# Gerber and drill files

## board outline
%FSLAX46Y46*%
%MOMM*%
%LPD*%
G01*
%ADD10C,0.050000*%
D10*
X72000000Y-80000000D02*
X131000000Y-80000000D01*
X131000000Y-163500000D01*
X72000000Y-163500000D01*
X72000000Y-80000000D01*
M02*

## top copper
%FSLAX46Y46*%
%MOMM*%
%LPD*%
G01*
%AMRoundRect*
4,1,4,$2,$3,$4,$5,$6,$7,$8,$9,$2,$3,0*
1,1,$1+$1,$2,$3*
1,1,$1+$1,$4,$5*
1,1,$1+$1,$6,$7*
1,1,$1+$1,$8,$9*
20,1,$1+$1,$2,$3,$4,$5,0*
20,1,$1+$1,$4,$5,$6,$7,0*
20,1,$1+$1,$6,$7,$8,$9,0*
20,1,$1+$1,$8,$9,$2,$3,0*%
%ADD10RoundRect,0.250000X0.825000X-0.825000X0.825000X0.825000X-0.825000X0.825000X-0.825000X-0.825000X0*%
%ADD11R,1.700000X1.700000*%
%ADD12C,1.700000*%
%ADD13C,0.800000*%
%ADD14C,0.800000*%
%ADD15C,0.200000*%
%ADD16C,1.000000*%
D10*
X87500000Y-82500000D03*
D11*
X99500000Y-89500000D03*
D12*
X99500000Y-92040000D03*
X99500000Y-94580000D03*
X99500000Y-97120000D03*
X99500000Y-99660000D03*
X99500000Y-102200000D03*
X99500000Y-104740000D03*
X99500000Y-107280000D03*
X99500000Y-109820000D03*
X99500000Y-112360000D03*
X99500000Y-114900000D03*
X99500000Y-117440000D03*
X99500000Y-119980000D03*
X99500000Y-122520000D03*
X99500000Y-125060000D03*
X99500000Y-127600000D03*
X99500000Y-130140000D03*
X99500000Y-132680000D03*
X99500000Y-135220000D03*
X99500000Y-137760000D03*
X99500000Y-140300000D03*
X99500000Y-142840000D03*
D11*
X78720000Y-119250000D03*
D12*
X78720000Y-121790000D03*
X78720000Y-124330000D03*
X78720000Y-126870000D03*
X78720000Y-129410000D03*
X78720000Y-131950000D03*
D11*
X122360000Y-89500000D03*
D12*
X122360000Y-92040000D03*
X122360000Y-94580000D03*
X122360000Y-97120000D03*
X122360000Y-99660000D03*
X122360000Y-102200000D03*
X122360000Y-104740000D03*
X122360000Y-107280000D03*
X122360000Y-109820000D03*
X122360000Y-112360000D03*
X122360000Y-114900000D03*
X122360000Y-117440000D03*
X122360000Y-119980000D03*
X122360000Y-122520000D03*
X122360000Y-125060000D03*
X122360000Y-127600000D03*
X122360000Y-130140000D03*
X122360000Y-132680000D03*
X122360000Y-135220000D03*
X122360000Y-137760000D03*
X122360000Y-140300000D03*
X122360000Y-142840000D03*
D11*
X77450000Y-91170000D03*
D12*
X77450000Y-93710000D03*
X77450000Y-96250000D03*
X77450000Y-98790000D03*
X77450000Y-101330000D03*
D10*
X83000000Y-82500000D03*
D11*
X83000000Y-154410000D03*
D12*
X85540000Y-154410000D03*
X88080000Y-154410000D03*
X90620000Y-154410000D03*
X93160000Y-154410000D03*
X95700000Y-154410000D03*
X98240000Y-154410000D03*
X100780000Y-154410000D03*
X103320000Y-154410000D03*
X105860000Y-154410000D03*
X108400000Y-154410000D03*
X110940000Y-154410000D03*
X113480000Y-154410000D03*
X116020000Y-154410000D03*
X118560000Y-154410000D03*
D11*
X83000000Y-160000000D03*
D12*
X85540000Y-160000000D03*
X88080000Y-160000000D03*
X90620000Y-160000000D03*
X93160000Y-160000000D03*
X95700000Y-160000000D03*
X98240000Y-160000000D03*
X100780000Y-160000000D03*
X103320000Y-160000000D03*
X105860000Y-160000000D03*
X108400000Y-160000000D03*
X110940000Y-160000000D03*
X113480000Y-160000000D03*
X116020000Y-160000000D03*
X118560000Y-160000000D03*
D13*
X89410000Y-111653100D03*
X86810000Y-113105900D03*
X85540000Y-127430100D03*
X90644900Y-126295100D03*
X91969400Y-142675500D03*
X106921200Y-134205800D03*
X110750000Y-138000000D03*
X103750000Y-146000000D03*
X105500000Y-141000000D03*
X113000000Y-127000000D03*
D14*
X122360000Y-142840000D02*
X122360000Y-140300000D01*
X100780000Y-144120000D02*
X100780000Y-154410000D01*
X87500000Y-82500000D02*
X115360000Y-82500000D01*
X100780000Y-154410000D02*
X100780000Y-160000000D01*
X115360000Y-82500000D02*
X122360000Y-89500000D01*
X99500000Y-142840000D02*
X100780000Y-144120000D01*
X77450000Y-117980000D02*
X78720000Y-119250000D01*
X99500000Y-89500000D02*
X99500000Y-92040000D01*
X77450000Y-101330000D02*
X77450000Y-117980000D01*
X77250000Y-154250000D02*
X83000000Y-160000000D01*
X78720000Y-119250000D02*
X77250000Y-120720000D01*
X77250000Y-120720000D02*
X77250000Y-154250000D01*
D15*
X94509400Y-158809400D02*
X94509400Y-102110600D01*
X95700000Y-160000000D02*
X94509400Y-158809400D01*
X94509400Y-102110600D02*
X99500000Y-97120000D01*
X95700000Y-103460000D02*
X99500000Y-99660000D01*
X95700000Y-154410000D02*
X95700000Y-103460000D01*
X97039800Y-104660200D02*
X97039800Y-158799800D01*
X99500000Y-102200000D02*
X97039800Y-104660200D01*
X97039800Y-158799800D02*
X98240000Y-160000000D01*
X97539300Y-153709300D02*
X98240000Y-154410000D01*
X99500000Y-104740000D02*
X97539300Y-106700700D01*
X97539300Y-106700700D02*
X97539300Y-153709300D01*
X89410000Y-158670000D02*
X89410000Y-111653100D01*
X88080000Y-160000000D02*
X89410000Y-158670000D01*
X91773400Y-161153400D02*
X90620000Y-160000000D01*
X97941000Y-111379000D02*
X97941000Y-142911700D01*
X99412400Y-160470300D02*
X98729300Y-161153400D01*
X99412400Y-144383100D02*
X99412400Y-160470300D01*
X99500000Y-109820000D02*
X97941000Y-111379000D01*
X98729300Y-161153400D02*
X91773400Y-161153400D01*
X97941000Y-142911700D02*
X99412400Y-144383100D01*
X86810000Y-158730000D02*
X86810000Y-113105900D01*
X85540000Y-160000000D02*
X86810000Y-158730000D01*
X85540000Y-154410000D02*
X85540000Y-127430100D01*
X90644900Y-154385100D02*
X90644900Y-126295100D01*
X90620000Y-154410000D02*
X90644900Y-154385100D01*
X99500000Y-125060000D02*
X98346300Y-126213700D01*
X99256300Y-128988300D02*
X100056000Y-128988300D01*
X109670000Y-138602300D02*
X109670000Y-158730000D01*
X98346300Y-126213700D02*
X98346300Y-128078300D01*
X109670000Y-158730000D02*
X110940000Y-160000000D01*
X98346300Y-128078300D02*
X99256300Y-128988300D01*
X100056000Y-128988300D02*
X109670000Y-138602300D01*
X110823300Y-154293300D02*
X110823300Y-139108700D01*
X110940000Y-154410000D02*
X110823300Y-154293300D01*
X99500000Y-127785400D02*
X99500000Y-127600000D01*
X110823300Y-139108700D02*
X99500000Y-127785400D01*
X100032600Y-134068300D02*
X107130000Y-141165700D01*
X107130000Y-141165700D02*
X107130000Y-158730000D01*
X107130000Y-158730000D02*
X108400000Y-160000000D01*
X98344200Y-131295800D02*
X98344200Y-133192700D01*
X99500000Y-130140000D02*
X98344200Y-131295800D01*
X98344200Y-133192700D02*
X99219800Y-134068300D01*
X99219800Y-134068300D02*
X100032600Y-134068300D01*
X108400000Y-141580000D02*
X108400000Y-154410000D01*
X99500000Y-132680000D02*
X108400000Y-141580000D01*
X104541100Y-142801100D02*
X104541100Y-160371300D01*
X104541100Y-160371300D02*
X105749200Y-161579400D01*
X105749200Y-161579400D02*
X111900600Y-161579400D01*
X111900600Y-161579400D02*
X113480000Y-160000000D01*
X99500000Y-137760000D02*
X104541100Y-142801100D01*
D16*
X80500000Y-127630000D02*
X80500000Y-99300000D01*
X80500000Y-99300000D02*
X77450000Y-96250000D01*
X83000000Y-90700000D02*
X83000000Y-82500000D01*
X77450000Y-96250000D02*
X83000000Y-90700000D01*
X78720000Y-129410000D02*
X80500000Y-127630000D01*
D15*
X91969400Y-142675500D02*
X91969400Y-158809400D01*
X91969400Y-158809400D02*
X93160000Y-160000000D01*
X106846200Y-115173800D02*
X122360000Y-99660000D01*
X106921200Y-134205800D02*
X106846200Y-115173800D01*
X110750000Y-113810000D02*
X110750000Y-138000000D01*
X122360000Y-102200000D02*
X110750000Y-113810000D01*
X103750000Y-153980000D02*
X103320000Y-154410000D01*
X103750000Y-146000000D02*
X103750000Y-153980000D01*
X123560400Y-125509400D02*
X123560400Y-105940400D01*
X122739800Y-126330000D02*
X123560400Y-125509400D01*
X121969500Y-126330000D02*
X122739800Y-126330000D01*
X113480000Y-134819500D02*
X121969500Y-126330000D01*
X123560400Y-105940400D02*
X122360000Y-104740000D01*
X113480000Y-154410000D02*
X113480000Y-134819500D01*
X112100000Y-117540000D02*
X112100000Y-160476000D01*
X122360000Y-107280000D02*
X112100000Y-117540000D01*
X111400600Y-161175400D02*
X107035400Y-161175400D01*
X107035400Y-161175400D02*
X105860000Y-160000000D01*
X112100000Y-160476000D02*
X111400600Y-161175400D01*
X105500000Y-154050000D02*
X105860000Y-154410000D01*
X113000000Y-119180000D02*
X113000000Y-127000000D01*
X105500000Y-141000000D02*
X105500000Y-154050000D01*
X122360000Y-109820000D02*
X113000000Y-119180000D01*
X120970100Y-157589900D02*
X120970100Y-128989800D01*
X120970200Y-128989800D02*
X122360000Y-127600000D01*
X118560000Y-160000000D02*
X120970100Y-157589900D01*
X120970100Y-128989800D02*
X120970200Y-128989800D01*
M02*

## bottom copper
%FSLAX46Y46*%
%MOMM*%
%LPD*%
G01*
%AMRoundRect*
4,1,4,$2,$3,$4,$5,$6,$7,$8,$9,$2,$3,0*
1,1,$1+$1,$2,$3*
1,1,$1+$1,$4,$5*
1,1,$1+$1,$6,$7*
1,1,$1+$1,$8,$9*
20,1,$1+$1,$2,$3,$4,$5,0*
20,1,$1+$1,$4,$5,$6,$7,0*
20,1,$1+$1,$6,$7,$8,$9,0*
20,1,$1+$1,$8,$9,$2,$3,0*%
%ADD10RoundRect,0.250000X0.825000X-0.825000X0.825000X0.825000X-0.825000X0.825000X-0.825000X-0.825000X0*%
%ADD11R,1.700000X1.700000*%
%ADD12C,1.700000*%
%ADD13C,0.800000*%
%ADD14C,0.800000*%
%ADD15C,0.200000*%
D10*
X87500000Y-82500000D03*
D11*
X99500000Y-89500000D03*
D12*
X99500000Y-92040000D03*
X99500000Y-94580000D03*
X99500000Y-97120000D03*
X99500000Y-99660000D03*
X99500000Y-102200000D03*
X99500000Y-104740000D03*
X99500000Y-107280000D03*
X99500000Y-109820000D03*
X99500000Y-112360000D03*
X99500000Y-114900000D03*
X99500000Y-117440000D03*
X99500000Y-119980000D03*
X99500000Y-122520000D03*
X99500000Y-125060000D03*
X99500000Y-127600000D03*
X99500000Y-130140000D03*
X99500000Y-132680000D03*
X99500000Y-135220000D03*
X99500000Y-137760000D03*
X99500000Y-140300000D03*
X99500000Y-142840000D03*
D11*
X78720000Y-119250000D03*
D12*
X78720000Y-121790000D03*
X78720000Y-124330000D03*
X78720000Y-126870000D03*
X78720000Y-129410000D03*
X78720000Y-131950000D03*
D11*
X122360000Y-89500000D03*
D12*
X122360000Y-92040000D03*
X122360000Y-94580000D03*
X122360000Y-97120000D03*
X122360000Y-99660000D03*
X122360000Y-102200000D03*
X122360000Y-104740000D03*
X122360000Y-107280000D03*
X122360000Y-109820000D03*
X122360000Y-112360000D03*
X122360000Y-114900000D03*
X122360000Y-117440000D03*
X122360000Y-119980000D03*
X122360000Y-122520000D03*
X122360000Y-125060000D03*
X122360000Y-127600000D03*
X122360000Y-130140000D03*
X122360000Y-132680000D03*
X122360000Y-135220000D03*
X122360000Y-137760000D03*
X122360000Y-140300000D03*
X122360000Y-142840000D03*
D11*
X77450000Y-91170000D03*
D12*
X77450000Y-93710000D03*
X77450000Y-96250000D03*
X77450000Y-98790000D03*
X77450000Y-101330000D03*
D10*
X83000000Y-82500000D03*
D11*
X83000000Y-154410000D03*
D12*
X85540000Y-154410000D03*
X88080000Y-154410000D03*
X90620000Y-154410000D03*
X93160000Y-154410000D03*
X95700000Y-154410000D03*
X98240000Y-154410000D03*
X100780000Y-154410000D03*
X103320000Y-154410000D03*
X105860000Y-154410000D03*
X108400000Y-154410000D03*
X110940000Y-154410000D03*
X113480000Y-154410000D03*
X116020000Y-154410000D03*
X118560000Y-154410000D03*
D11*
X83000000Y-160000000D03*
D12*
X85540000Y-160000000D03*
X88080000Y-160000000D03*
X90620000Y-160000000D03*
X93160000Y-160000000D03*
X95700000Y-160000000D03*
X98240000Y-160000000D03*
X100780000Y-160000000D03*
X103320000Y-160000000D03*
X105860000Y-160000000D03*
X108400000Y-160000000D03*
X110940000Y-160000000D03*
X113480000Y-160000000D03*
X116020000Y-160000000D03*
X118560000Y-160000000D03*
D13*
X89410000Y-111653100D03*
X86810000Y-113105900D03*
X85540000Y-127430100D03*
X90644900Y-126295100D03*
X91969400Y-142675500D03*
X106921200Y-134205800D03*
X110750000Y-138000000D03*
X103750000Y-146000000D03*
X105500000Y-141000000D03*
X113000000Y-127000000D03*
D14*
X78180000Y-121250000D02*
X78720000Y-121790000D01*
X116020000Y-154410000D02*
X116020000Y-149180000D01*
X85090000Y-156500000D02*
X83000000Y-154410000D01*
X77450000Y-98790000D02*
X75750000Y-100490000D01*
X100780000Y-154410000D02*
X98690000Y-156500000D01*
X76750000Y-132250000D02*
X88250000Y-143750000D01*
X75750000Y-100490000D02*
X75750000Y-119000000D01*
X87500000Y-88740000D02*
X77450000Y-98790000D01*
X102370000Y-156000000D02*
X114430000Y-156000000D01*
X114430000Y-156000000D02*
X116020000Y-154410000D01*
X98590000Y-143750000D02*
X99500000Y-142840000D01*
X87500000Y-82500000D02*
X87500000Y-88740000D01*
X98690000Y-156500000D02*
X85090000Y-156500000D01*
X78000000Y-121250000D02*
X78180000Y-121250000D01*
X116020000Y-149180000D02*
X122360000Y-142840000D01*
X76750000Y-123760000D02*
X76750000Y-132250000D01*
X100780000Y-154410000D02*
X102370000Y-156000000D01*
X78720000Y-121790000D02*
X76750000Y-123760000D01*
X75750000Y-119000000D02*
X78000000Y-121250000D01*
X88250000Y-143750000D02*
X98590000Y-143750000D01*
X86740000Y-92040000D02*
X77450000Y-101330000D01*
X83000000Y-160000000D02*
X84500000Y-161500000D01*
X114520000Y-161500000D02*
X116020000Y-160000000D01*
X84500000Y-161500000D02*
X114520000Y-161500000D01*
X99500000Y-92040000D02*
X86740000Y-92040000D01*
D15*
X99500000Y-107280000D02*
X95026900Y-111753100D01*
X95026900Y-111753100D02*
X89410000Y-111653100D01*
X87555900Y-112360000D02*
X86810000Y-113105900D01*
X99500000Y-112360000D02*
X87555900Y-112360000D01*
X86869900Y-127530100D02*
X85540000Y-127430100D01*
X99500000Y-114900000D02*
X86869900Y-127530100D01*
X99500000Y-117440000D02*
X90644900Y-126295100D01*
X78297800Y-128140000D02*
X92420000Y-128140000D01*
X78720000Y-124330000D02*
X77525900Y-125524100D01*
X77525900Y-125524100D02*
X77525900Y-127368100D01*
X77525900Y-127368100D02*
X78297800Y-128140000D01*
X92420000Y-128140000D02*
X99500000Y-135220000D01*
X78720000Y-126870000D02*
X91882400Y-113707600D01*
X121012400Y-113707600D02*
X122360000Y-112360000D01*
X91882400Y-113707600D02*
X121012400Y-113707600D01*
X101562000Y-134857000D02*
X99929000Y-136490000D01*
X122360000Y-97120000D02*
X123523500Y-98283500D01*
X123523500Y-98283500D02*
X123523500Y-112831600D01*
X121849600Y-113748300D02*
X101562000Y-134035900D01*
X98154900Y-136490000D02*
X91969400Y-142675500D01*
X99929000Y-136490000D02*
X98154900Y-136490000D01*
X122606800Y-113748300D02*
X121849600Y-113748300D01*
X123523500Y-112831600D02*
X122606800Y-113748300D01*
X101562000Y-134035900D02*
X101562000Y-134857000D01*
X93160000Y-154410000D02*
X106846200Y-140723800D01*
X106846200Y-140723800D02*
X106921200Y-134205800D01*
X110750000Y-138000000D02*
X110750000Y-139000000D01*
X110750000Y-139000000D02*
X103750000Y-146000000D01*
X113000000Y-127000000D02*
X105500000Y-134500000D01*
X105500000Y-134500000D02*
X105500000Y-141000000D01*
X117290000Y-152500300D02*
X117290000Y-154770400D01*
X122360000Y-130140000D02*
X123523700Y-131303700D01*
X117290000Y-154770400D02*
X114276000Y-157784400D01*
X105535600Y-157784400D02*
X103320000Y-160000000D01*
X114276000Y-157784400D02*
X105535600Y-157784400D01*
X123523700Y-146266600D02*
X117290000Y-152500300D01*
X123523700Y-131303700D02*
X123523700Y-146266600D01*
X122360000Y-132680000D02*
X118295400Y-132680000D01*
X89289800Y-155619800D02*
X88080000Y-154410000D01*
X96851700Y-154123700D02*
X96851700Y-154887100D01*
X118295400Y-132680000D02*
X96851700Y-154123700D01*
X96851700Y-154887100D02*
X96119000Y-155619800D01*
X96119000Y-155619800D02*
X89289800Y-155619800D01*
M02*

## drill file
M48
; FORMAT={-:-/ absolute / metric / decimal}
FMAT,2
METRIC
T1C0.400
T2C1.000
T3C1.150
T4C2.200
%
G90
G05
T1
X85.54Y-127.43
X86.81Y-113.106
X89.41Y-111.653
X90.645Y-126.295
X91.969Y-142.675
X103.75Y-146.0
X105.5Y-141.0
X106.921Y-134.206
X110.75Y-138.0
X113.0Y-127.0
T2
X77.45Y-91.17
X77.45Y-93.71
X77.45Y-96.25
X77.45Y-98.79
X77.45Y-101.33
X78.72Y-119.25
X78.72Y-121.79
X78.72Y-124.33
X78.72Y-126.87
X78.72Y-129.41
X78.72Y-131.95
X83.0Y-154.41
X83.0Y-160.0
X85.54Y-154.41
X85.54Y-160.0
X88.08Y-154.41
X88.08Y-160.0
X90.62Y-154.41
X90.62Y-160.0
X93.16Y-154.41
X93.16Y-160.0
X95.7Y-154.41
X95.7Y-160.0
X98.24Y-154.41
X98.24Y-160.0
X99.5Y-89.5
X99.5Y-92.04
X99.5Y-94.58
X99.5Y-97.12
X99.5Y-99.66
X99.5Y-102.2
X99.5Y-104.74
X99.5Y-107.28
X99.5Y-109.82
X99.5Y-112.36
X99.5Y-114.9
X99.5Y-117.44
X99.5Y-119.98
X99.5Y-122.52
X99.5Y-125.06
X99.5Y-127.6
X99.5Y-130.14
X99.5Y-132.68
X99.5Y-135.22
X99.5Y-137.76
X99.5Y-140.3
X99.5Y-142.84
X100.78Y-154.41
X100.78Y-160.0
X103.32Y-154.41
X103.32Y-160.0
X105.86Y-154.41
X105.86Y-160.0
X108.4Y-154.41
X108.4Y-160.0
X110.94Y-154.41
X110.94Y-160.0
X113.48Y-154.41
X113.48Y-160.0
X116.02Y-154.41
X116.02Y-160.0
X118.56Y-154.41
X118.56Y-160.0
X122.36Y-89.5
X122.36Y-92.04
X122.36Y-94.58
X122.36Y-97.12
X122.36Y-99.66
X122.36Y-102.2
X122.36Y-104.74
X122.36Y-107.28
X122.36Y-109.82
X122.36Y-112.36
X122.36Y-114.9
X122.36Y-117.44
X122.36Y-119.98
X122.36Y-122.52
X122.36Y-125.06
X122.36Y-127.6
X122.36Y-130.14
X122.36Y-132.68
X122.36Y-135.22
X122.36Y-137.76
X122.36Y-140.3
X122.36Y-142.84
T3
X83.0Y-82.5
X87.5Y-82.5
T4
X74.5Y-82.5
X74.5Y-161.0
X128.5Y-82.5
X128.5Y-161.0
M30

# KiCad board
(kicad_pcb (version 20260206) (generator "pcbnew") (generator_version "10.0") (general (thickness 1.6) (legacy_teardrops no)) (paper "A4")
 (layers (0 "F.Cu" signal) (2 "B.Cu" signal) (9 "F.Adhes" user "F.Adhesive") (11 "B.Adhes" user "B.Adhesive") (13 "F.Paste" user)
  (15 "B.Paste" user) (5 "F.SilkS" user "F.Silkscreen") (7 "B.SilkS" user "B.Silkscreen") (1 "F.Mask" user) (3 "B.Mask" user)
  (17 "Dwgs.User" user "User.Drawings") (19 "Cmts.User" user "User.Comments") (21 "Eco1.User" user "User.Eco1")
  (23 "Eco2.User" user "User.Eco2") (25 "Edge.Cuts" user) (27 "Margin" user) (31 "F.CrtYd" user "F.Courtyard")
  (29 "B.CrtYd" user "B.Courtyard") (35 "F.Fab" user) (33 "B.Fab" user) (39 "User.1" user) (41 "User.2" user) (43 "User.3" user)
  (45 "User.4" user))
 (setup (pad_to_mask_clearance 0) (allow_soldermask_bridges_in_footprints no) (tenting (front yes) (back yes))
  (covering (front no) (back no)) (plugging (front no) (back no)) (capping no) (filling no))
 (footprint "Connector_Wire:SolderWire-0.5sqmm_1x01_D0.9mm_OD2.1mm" (layer "F.Cu") (at 87.5 82.5 90)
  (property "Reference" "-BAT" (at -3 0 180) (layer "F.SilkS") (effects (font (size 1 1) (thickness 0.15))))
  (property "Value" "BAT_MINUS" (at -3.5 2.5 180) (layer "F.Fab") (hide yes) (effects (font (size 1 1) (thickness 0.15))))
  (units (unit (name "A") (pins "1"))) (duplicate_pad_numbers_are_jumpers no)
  (pad "1" thru_hole roundrect (at 0 0 90) (size 2.15 2.15) (drill 1.15) (layers "*.Cu" "*.Mask") (remove_unused_layers no)
   (roundrect_rratio 0.116279) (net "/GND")))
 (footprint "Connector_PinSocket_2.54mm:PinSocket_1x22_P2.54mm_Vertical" (layer "F.Cu") (at 99.5 89.5)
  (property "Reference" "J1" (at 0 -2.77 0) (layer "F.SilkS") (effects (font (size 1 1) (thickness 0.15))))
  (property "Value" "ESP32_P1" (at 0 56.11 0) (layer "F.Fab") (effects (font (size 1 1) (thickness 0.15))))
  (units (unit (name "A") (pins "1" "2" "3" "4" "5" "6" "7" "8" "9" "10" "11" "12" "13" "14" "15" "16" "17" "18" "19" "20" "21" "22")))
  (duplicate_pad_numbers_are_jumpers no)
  (pad "1" thru_hole rect (at 0 0) (size 1.7 1.7) (drill 1) (layers "*.Cu" "*.Mask") (remove_unused_layers no) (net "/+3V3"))
  (pad "2" thru_hole circle (at 0 2.54) (size 1.7 1.7) (drill 1) (layers "*.Cu" "*.Mask") (remove_unused_layers no) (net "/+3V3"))
  (pad "3" thru_hole circle (at 0 5.08) (size 1.7 1.7) (drill 1) (layers "*.Cu" "*.Mask") (remove_unused_layers no) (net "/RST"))
  (pad "4" thru_hole circle (at 0 7.62) (size 1.7 1.7) (drill 1) (layers "*.Cu" "*.Mask") (remove_unused_layers no) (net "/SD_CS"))
  (pad "5" thru_hole circle (at 0 10.16) (size 1.7 1.7) (drill 1) (layers "*.Cu" "*.Mask") (remove_unused_layers no) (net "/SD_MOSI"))
  (pad "6" thru_hole circle (at 0 12.7) (size 1.7 1.7) (drill 1) (layers "*.Cu" "*.Mask") (remove_unused_layers no) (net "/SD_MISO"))
  (pad "7" thru_hole circle (at 0 15.24) (size 1.7 1.7) (drill 1) (layers "*.Cu" "*.Mask") (remove_unused_layers no) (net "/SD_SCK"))
  (pad "8" thru_hole circle (at 0 17.78) (size 1.7 1.7) (drill 1) (layers "*.Cu" "*.Mask") (remove_unused_layers no) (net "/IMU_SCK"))
  (pad "9" thru_hole circle (at 0 20.32) (size 1.7 1.7) (drill 1) (layers "*.Cu" "*.Mask") (remove_unused_layers no) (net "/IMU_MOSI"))
  (pad "10" thru_hole circle (at 0 22.86) (size 1.7 1.7) (drill 1) (layers "*.Cu" "*.Mask") (remove_unused_layers no) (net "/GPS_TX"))
  (pad "11" thru_hole circle (at 0 25.4) (size 1.7 1.7) (drill 1) (layers "*.Cu" "*.Mask") (remove_unused_layers no) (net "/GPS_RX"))
  (pad "12" thru_hole circle (at 0 27.94) (size 1.7 1.7) (drill 1) (layers "*.Cu" "*.Mask") (remove_unused_layers no) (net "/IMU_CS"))
  (pad "13" thru_hole circle (at 0 30.48) (size 1.7 1.7) (drill 1) (layers "*.Cu" "*.Mask") (remove_unused_layers no) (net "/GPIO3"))
  (pad "14" thru_hole circle (at 0 33.02) (size 1.7 1.7) (drill 1) (layers "*.Cu" "*.Mask") (remove_unused_layers no) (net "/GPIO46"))
  (pad "15" thru_hole circle (at 0 35.56) (size 1.7 1.7) (drill 1) (layers "*.Cu" "*.Mask") (remove_unused_layers no) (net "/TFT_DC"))
  (pad "16" thru_hole circle (at 0 38.1) (size 1.7 1.7) (drill 1) (layers "*.Cu" "*.Mask") (remove_unused_layers no) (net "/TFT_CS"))
  (pad "17" thru_hole circle (at 0 40.64) (size 1.7 1.7) (drill 1) (layers "*.Cu" "*.Mask") (remove_unused_layers no) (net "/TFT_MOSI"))
  (pad "18" thru_hole circle (at 0 43.18) (size 1.7 1.7) (drill 1) (layers "*.Cu" "*.Mask") (remove_unused_layers no) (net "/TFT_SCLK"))
  (pad "19" thru_hole circle (at 0 45.72) (size 1.7 1.7) (drill 1) (layers "*.Cu" "*.Mask") (remove_unused_layers no) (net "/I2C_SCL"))
  (pad "20" thru_hole circle (at 0 48.26) (size 1.7 1.7) (drill 1) (layers "*.Cu" "*.Mask") (remove_unused_layers no) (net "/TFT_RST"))
  (pad "21" thru_hole circle (at 0 50.8) (size 1.7 1.7) (drill 1) (layers "*.Cu" "*.Mask") (remove_unused_layers no) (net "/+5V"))
  (pad "22" thru_hole circle (at 0 53.34) (size 1.7 1.7) (drill 1) (layers "*.Cu" "*.Mask") (remove_unused_layers no) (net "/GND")))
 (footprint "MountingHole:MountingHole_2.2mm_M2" (layer "F.Cu") (at 74.5 82.5)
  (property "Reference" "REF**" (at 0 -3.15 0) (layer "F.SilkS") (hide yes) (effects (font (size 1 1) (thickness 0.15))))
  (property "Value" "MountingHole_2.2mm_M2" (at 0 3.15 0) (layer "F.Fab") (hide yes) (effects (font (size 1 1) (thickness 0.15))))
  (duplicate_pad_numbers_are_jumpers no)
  (pad "" np_thru_hole circle (at 0 0) (size 2.2 2.2) (drill 2.2) (layers "*.Cu" "*.Mask")))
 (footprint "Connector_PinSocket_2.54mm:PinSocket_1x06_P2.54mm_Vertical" (layer "F.Cu") (at 78.72 119.25)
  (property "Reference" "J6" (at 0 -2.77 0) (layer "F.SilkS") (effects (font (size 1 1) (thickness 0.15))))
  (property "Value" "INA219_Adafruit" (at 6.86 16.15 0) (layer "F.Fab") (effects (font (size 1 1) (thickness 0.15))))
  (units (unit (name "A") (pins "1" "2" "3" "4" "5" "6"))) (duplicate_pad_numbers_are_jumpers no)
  (pad "1" thru_hole rect (at 0 0) (size 1.7 1.7) (drill 1) (layers "*.Cu" "*.Mask") (remove_unused_layers no) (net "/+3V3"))
  (pad "2" thru_hole circle (at 0 2.54) (size 1.7 1.7) (drill 1) (layers "*.Cu" "*.Mask") (remove_unused_layers no) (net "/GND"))
  (pad "3" thru_hole circle (at 0 5.08) (size 1.7 1.7) (drill 1) (layers "*.Cu" "*.Mask") (remove_unused_layers no) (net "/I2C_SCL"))
  (pad "4" thru_hole circle (at 0 7.62) (size 1.7 1.7) (drill 1) (layers "*.Cu" "*.Mask") (remove_unused_layers no) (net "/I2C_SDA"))
  (pad "5" thru_hole circle (at 0 10.16) (size 1.7 1.7) (drill 1) (layers "*.Cu" "*.Mask") (remove_unused_layers no) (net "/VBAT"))
  (pad "6" thru_hole circle (at 0 12.7) (size 1.7 1.7) (drill 1) (layers "*.Cu" "*.Mask") (remove_unused_layers no)
   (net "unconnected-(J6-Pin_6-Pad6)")))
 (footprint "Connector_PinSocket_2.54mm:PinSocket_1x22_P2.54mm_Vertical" (layer "F.Cu") (at 122.36 89.5)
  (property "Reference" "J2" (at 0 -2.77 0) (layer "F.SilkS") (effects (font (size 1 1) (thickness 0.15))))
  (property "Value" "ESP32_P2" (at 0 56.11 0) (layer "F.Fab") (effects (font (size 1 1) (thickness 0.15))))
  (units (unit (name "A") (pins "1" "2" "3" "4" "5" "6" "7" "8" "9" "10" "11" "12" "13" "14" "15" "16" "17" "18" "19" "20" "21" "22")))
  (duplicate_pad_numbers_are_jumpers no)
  (pad "1" thru_hole rect (at 0 0) (size 1.7 1.7) (drill 1) (layers "*.Cu" "*.Mask") (remove_unused_layers no) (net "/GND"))
  (pad "2" thru_hole circle (at 0 2.54) (size 1.7 1.7) (drill 1) (layers "*.Cu" "*.Mask") (remove_unused_layers no) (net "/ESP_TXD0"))
  (pad "3" thru_hole circle (at 0 5.08) (size 1.7 1.7) (drill 1) (layers "*.Cu" "*.Mask") (remove_unused_layers no) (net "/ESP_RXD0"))
  (pad "4" thru_hole circle (at 0 7.62) (size 1.7 1.7) (drill 1) (layers "*.Cu" "*.Mask") (remove_unused_layers no) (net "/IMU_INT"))
  (pad "5" thru_hole circle (at 0 10.16) (size 1.7 1.7) (drill 1) (layers "*.Cu" "*.Mask") (remove_unused_layers no) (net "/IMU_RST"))
  (pad "6" thru_hole circle (at 0 12.7) (size 1.7 1.7) (drill 1) (layers "*.Cu" "*.Mask") (remove_unused_layers no) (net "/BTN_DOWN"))
  (pad "7" thru_hole circle (at 0 15.24) (size 1.7 1.7) (drill 1) (layers "*.Cu" "*.Mask") (remove_unused_layers no) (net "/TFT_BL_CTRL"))
  (pad "8" thru_hole circle (at 0 17.78) (size 1.7 1.7) (drill 1) (layers "*.Cu" "*.Mask") (remove_unused_layers no) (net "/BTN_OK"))
  (pad "9" thru_hole circle (at 0 20.32) (size 1.7 1.7) (drill 1) (layers "*.Cu" "*.Mask") (remove_unused_layers no) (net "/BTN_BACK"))
  (pad "10" thru_hole circle (at 0 22.86) (size 1.7 1.7) (drill 1) (layers "*.Cu" "*.Mask") (remove_unused_layers no) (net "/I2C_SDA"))
  (pad "11" thru_hole circle (at 0 25.4) (size 1.7 1.7) (drill 1) (layers "*.Cu" "*.Mask") (remove_unused_layers no) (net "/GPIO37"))
  (pad "12" thru_hole circle (at 0 27.94) (size 1.7 1.7) (drill 1) (layers "*.Cu" "*.Mask") (remove_unused_layers no) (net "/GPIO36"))
  (pad "13" thru_hole circle (at 0 30.48) (size 1.7 1.7) (drill 1) (layers "*.Cu" "*.Mask") (remove_unused_layers no) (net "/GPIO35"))
  (pad "14" thru_hole circle (at 0 33.02) (size 1.7 1.7) (drill 1) (layers "*.Cu" "*.Mask") (remove_unused_layers no) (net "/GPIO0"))
  (pad "15" thru_hole circle (at 0 35.56) (size 1.7 1.7) (drill 1) (layers "*.Cu" "*.Mask") (remove_unused_layers no) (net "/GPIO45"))
  (pad "16" thru_hole circle (at 0 38.1) (size 1.7 1.7) (drill 1) (layers "*.Cu" "*.Mask") (remove_unused_layers no) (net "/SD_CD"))
  (pad "17" thru_hole circle (at 0 40.64) (size 1.7 1.7) (drill 1) (layers "*.Cu" "*.Mask") (remove_unused_layers no) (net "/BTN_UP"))
  (pad "18" thru_hole circle (at 0 43.18) (size 1.7 1.7) (drill 1) (layers "*.Cu" "*.Mask") (remove_unused_layers no) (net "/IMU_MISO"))
  (pad "19" thru_hole circle (at 0 45.72) (size 1.7 1.7) (drill 1) (layers "*.Cu" "*.Mask") (remove_unused_layers no) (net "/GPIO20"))
  (pad "20" thru_hole circle (at 0 48.26) (size 1.7 1.7) (drill 1) (layers "*.Cu" "*.Mask") (remove_unused_layers no) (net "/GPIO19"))
  (pad "21" thru_hole circle (at 0 50.8) (size 1.7 1.7) (drill 1) (layers "*.Cu" "*.Mask") (remove_unused_layers no) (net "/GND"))
  (pad "22" thru_hole circle (at 0 53.34) (size 1.7 1.7) (drill 1) (layers "*.Cu" "*.Mask") (remove_unused_layers no) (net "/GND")))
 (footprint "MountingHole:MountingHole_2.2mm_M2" (layer "F.Cu") (at 74.5 161)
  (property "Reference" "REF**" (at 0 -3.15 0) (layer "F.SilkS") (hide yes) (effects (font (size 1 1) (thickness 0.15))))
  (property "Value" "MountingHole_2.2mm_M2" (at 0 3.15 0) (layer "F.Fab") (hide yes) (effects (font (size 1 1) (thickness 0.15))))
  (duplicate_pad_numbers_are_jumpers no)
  (pad "" np_thru_hole circle (at 0 0) (size 2.2 2.2) (drill 2.2) (layers "*.Cu" "*.Mask")))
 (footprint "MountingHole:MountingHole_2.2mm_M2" (layer "F.Cu") (at 128.5 82.5)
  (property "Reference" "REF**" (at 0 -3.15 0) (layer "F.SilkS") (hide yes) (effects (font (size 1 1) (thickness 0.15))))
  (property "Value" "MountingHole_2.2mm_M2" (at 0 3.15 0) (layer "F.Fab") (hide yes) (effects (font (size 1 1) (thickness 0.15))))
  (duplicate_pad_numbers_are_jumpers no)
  (pad "" np_thru_hole circle (at 0 0) (size 2.2 2.2) (drill 2.2) (layers "*.Cu" "*.Mask")))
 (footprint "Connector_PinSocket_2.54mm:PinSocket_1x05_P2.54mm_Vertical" (layer "F.Cu") (at 77.45 91.17)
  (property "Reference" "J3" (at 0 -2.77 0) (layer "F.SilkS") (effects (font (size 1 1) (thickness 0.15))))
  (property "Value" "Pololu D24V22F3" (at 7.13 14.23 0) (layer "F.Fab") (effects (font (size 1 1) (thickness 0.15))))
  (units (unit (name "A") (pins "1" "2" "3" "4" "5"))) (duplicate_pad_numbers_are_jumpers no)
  (pad "1" thru_hole rect (at 0 0) (size 1.7 1.7) (drill 1) (layers "*.Cu" "*.Mask") (remove_unused_layers no)
   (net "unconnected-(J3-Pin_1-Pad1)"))
  (pad "2" thru_hole circle (at 0 2.54) (size 1.7 1.7) (drill 1) (layers "*.Cu" "*.Mask") (remove_unused_layers no)
   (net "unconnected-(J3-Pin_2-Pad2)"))
  (pad "3" thru_hole circle (at 0 5.08) (size 1.7 1.7) (drill 1) (layers "*.Cu" "*.Mask") (remove_unused_layers no) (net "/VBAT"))
  (pad "4" thru_hole circle (at 0 7.62) (size 1.7 1.7) (drill 1) (layers "*.Cu" "*.Mask") (remove_unused_layers no) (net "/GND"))
  (pad "5" thru_hole circle (at 0 10.16) (size 1.7 1.7) (drill 1) (layers "*.Cu" "*.Mask") (remove_unused_layers no) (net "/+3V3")))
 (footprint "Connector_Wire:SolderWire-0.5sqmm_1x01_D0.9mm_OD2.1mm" (layer "F.Cu") (at 83 82.5 90)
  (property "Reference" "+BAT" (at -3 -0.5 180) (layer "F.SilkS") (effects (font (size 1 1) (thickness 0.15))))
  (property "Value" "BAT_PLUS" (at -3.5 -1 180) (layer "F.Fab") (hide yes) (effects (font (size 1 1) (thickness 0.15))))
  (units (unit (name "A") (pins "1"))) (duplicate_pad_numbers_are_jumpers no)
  (pad "1" thru_hole roundrect (at 0 0 90) (size 2.15 2.15) (drill 1.15) (layers "*.Cu" "*.Mask") (remove_unused_layers no)
   (roundrect_rratio 0.116279) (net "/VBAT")))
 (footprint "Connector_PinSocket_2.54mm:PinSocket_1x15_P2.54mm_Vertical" (layer "F.Cu") (at 83 154.41 90)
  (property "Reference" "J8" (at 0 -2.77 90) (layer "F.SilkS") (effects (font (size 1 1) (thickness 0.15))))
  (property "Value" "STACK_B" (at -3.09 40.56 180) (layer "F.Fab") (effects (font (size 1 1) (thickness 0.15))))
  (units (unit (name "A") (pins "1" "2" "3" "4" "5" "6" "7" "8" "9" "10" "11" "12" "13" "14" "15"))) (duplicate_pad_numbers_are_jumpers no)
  (pad "1" thru_hole rect (at 0 0 90) (size 1.7 1.7) (drill 1) (layers "*.Cu" "*.Mask") (remove_unused_layers no) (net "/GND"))
  (pad "2" thru_hole circle (at 0 2.54 90) (size 1.7 1.7) (drill 1) (layers "*.Cu" "*.Mask") (remove_unused_layers no) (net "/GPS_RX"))
  (pad "3" thru_hole circle (at 0 5.08 90) (size 1.7 1.7) (drill 1) (layers "*.Cu" "*.Mask") (remove_unused_layers no) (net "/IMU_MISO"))
  (pad "4" thru_hole circle (at 0 7.62 90) (size 1.7 1.7) (drill 1) (layers "*.Cu" "*.Mask") (remove_unused_layers no) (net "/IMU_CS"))
  (pad "5" thru_hole circle (at 0 10.16 90) (size 1.7 1.7) (drill 1) (layers "*.Cu" "*.Mask") (remove_unused_layers no) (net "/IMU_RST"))
  (pad "6" thru_hole circle (at 0 12.7 90) (size 1.7 1.7) (drill 1) (layers "*.Cu" "*.Mask") (remove_unused_layers no) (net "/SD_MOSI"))
  (pad "7" thru_hole circle (at 0 15.24 90) (size 1.7 1.7) (drill 1) (layers "*.Cu" "*.Mask") (remove_unused_layers no) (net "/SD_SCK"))
  (pad "8" thru_hole circle (at 0 17.78 90) (size 1.7 1.7) (drill 1) (layers "*.Cu" "*.Mask") (remove_unused_layers no) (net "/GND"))
  (pad "9" thru_hole circle (at 0 20.32 90) (size 1.7 1.7) (drill 1) (layers "*.Cu" "*.Mask") (remove_unused_layers no) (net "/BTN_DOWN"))
  (pad "10" thru_hole circle (at 0 22.86 90) (size 1.7 1.7) (drill 1) (layers "*.Cu" "*.Mask") (remove_unused_layers no) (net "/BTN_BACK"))
  (pad "11" thru_hole circle (at 0 25.4 90) (size 1.7 1.7) (drill 1) (layers "*.Cu" "*.Mask") (remove_unused_layers no) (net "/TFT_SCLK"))
  (pad "12" thru_hole circle (at 0 27.94 90) (size 1.7 1.7) (drill 1) (layers "*.Cu" "*.Mask") (remove_unused_layers no) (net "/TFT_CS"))
  (pad "13" thru_hole circle (at 0 30.48 90) (size 1.7 1.7) (drill 1) (layers "*.Cu" "*.Mask") (remove_unused_layers no)
   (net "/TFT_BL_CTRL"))
  (pad "14" thru_hole circle (at 0 33.02 90) (size 1.7 1.7) (drill 1) (layers "*.Cu" "*.Mask") (remove_unused_layers no) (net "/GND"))
  (pad "15" thru_hole circle (at 0 35.56 90) (size 1.7 1.7) (drill 1) (layers "*.Cu" "*.Mask") (remove_unused_layers no)
   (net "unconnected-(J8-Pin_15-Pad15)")))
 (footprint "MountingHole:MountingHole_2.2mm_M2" (layer "F.Cu") (at 128.5 161)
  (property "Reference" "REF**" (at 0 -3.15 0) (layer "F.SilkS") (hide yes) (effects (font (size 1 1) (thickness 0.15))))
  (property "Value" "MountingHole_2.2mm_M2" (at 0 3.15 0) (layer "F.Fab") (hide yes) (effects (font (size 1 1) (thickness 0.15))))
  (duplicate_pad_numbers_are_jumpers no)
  (pad "" np_thru_hole circle (at 0 0) (size 2.2 2.2) (drill 2.2) (layers "*.Cu" "*.Mask")))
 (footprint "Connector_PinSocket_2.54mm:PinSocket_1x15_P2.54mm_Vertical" (layer "F.Cu") (at 83 160 90)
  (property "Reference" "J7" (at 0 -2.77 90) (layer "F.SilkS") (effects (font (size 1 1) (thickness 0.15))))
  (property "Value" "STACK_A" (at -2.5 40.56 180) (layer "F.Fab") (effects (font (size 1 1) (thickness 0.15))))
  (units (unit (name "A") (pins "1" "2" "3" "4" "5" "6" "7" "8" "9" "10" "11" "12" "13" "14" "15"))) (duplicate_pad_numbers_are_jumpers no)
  (pad "1" thru_hole rect (at 0 0 90) (size 1.7 1.7) (drill 1) (layers "*.Cu" "*.Mask") (remove_unused_layers no) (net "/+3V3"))
  (pad "2" thru_hole circle (at 0 2.54 90) (size 1.7 1.7) (drill 1) (layers "*.Cu" "*.Mask") (remove_unused_layers no) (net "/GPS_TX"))
  (pad "3" thru_hole circle (at 0 5.08 90) (size 1.7 1.7) (drill 1) (layers "*.Cu" "*.Mask") (remove_unused_layers no) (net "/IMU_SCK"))
  (pad "4" thru_hole circle (at 0 7.62 90) (size 1.7 1.7) (drill 1) (layers "*.Cu" "*.Mask") (remove_unused_layers no) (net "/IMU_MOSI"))
  (pad "5" thru_hole circle (at 0 10.16 90) (size 1.7 1.7) (drill 1) (layers "*.Cu" "*.Mask") (remove_unused_layers no) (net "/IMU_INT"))
  (pad "6" thru_hole circle (at 0 12.7 90) (size 1.7 1.7) (drill 1) (layers "*.Cu" "*.Mask") (remove_unused_layers no) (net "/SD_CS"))
  (pad "7" thru_hole circle (at 0 15.24 90) (size 1.7 1.7) (drill 1) (layers "*.Cu" "*.Mask") (remove_unused_layers no) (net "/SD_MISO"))
  (pad "8" thru_hole circle (at 0 17.78 90) (size 1.7 1.7) (drill 1) (layers "*.Cu" "*.Mask") (remove_unused_layers no) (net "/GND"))
  (pad "9" thru_hole circle (at 0 20.32 90) (size 1.7 1.7) (drill 1) (layers "*.Cu" "*.Mask") (remove_unused_layers no) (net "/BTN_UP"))
  (pad "10" thru_hole circle (at 0 22.86 90) (size 1.7 1.7) (drill 1) (layers "*.Cu" "*.Mask") (remove_unused_layers no) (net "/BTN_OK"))
  (pad "11" thru_hole circle (at 0 25.4 90) (size 1.7 1.7) (drill 1) (layers "*.Cu" "*.Mask") (remove_unused_layers no) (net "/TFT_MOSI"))
  (pad "12" thru_hole circle (at 0 27.94 90) (size 1.7 1.7) (drill 1) (layers "*.Cu" "*.Mask") (remove_unused_layers no) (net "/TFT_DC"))
  (pad "13" thru_hole circle (at 0 30.48 90) (size 1.7 1.7) (drill 1) (layers "*.Cu" "*.Mask") (remove_unused_layers no) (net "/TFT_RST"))
  (pad "14" thru_hole circle (at 0 33.02 90) (size 1.7 1.7) (drill 1) (layers "*.Cu" "*.Mask") (remove_unused_layers no) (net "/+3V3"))
  (pad "15" thru_hole circle (at 0 35.56 90) (size 1.7 1.7) (drill 1) (layers "*.Cu" "*.Mask") (remove_unused_layers no) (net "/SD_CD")))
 (gr_rect (start 72 80) (end 131 163.5) (stroke (width 0.05) (type default)) (fill no) (layer "Edge.Cuts"))
 (segment (start 122.36 142.84) (end 122.36 140.3) (width 0.8) (layer "F.Cu") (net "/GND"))
 (segment (start 100.78 144.12) (end 100.78 154.41) (width 0.8) (layer "F.Cu") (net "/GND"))
 (segment (start 87.5 82.5) (end 115.36 82.5) (width 0.8) (layer "F.Cu") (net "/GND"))
 (segment (start 100.78 154.41) (end 100.78 160) (width 0.8) (layer "F.Cu") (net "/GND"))
 (segment (start 115.36 82.5) (end 122.36 89.5) (width 0.8) (layer "F.Cu") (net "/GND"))
 (segment (start 99.5 142.84) (end 100.78 144.12) (width 0.8) (layer "F.Cu") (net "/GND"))
 (segment (start 78.18 121.25) (end 78.72 121.79) (width 0.8) (layer "B.Cu") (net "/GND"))
 (segment (start 116.02 154.41) (end 116.02 149.18) (width 0.8) (layer "B.Cu") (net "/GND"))
 (segment (start 85.09 156.5) (end 83 154.41) (width 0.8) (layer "B.Cu") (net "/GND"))
 (segment (start 77.45 98.79) (end 75.75 100.49) (width 0.8) (layer "B.Cu") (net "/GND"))
 (segment (start 100.78 154.41) (end 98.69 156.5) (width 0.8) (layer "B.Cu") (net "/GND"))
 (segment (start 76.75 132.25) (end 88.25 143.75) (width 0.8) (layer "B.Cu") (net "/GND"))
 (segment (start 75.75 100.49) (end 75.75 119) (width 0.8) (layer "B.Cu") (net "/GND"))
 (segment (start 87.5 88.74) (end 77.45 98.79) (width 0.8) (layer "B.Cu") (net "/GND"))
 (segment (start 102.37 156) (end 114.43 156) (width 0.8) (layer "B.Cu") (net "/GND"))
 (segment (start 114.43 156) (end 116.02 154.41) (width 0.8) (layer "B.Cu") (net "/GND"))
 (segment (start 98.59 143.75) (end 99.5 142.84) (width 0.8) (layer "B.Cu") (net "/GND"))
 (segment (start 87.5 82.5) (end 87.5 88.74) (width 0.8) (layer "B.Cu") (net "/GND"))
 (segment (start 98.69 156.5) (end 85.09 156.5) (width 0.8) (layer "B.Cu") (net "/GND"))
 (segment (start 78 121.25) (end 78.18 121.25) (width 0.8) (layer "B.Cu") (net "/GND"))
 (segment (start 116.02 149.18) (end 122.36 142.84) (width 0.8) (layer "B.Cu") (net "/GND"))
 (segment (start 76.75 123.76) (end 76.75 132.25) (width 0.8) (layer "B.Cu") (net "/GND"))
 (segment (start 100.78 154.41) (end 102.37 156) (width 0.8) (layer "B.Cu") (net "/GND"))
 (segment (start 78.72 121.79) (end 76.75 123.76) (width 0.8) (layer "B.Cu") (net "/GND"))
 (segment (start 75.75 119) (end 78 121.25) (width 0.8) (layer "B.Cu") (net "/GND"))
 (segment (start 88.25 143.75) (end 98.59 143.75) (width 0.8) (layer "B.Cu") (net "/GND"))
 (segment (start 77.45 117.98) (end 78.72 119.25) (width 0.8) (layer "F.Cu") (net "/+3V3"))
 (segment (start 99.5 89.5) (end 99.5 92.04) (width 0.8) (layer "F.Cu") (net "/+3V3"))
 (segment (start 77.45 101.33) (end 77.45 117.98) (width 0.8) (layer "F.Cu") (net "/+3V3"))
 (segment (start 77.25 154.25) (end 83 160) (width 0.8) (layer "F.Cu") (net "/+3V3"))
 (segment (start 78.72 119.25) (end 77.25 120.72) (width 0.8) (layer "F.Cu") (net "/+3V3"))
 (segment (start 77.25 120.72) (end 77.25 154.25) (width 0.8) (layer "F.Cu") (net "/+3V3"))
 (segment (start 86.74 92.04) (end 77.45 101.33) (width 0.8) (layer "B.Cu") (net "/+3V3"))
 (segment (start 83 160) (end 84.5 161.5) (width 0.8) (layer "B.Cu") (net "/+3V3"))
 (segment (start 114.52 161.5) (end 116.02 160) (width 0.8) (layer "B.Cu") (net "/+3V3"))
 (segment (start 84.5 161.5) (end 114.52 161.5) (width 0.8) (layer "B.Cu") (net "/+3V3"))
 (segment (start 99.5 92.04) (end 86.74 92.04) (width 0.8) (layer "B.Cu") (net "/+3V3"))
 (segment (start 94.5094 158.8094) (end 94.5094 102.1106) (width 0.2) (layer "F.Cu") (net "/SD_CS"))
 (segment (start 95.7 160) (end 94.5094 158.8094) (width 0.2) (layer "F.Cu") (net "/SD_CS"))
 (segment (start 94.5094 102.1106) (end 99.5 97.12) (width 0.2) (layer "F.Cu") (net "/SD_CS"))
 (segment (start 95.7 103.46) (end 99.5 99.66) (width 0.2) (layer "F.Cu") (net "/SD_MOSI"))
 (segment (start 95.7 154.41) (end 95.7 103.46) (width 0.2) (layer "F.Cu") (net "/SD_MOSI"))
 (segment (start 97.0398 104.6602) (end 97.0398 158.7998) (width 0.2) (layer "F.Cu") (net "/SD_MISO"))
 (segment (start 99.5 102.2) (end 97.0398 104.6602) (width 0.2) (layer "F.Cu") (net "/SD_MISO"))
 (segment (start 97.0398 158.7998) (end 98.24 160) (width 0.2) (layer "F.Cu") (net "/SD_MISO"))
 (segment (start 97.5393 153.7093) (end 98.24 154.41) (width 0.2) (layer "F.Cu") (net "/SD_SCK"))
 (segment (start 99.5 104.74) (end 97.5393 106.7007) (width 0.2) (layer "F.Cu") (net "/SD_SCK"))
 (segment (start 97.5393 106.7007) (end 97.5393 153.7093) (width 0.2) (layer "F.Cu") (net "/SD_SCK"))
 (segment (start 89.41 158.67) (end 89.41 111.6531) (width 0.2) (layer "F.Cu") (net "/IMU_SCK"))
 (segment (start 88.08 160) (end 89.41 158.67) (width 0.2) (layer "F.Cu") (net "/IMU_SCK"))
 (via (at 89.41 111.6531) (size 0.8) (drill 0.4) (layers "F.Cu" "B.Cu") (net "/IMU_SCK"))
 (segment (start 99.5 107.28) (end 95.0269 111.7531) (width 0.2) (layer "B.Cu") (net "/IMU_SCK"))
 (segment (start 95.0269 111.7531) (end 89.41 111.6531) (width 0.2) (layer "B.Cu") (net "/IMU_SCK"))
 (segment (start 91.7734 161.1534) (end 90.62 160) (width 0.2) (layer "F.Cu") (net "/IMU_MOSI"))
 (segment (start 97.941 111.379) (end 97.941 142.9117) (width 0.2) (layer "F.Cu") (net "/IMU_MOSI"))
 (segment (start 99.4124 160.4703) (end 98.7293 161.1534) (width 0.2) (layer "F.Cu") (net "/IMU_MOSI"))
 (segment (start 99.4124 144.3831) (end 99.4124 160.4703) (width 0.2) (layer "F.Cu") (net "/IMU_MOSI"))
 (segment (start 99.5 109.82) (end 97.941 111.379) (width 0.2) (layer "F.Cu") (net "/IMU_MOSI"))
 (segment (start 98.7293 161.1534) (end 91.7734 161.1534) (width 0.2) (layer "F.Cu") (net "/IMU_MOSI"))
 (segment (start 97.941 142.9117) (end 99.4124 144.3831) (width 0.2) (layer "F.Cu") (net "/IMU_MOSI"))
 (segment (start 86.81 158.73) (end 86.81 113.1059) (width 0.2) (layer "F.Cu") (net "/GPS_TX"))
 (segment (start 85.54 160) (end 86.81 158.73) (width 0.2) (layer "F.Cu") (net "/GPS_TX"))
 (via (at 86.81 113.1059) (size 0.8) (drill 0.4) (layers "F.Cu" "B.Cu") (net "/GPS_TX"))
 (segment (start 87.5559 112.36) (end 86.81 113.1059) (width 0.2) (layer "B.Cu") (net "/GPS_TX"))
 (segment (start 99.5 112.36) (end 87.5559 112.36) (width 0.2) (layer "B.Cu") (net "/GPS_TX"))
 (segment (start 85.54 154.41) (end 85.54 127.4301) (width 0.2) (layer "F.Cu") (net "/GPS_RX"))
 (via (at 85.54 127.4301) (size 0.8) (drill 0.4) (layers "F.Cu" "B.Cu") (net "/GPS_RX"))
 (segment (start 86.8699 127.5301) (end 85.54 127.4301) (width 0.2) (layer "B.Cu") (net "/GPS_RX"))
 (segment (start 99.5 114.9) (end 86.8699 127.5301) (width 0.2) (layer "B.Cu") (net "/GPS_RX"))
 (segment (start 90.6449 154.3851) (end 90.6449 126.2951) (width 0.2) (layer "F.Cu") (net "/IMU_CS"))
 (segment (start 90.62 154.41) (end 90.6449 154.3851) (width 0.2) (layer "F.Cu") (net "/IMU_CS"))
 (via (at 90.6449 126.2951) (size 0.8) (drill 0.4) (layers "F.Cu" "B.Cu") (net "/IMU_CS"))
 (segment (start 99.5 117.44) (end 90.6449 126.2951) (width 0.2) (layer "B.Cu") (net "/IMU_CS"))
 (segment (start 99.5 125.06) (end 98.3463 126.2137) (width 0.2) (layer "F.Cu") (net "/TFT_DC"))
 (segment (start 99.2563 128.9883) (end 100.056 128.9883) (width 0.2) (layer "F.Cu") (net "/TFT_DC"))
 (segment (start 109.67 138.6023) (end 109.67 158.73) (width 0.2) (layer "F.Cu") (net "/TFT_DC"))
 (segment (start 98.3463 126.2137) (end 98.3463 128.0783) (width 0.2) (layer "F.Cu") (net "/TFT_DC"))
 (segment (start 109.67 158.73) (end 110.94 160) (width 0.2) (layer "F.Cu") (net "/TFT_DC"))
 (segment (start 98.3463 128.0783) (end 99.2563 128.9883) (width 0.2) (layer "F.Cu") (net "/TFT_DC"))
 (segment (start 100.056 128.9883) (end 109.67 138.6023) (width 0.2) (layer "F.Cu") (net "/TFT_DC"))
 (segment (start 110.8233 154.2933) (end 110.8233 139.1087) (width 0.2) (layer "F.Cu") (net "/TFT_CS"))
 (segment (start 110.94 154.41) (end 110.8233 154.2933) (width 0.2) (layer "F.Cu") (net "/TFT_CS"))
 (segment (start 99.5 127.7854) (end 99.5 127.6) (width 0.2) (layer "F.Cu") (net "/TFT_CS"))
 (segment (start 110.8233 139.1087) (end 99.5 127.7854) (width 0.2) (layer "F.Cu") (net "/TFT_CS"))
 (segment (start 100.0326 134.0683) (end 107.13 141.1657) (width 0.2) (layer "F.Cu") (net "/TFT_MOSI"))
 (segment (start 107.13 141.1657) (end 107.13 158.73) (width 0.2) (layer "F.Cu") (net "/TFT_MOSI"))
 (segment (start 107.13 158.73) (end 108.4 160) (width 0.2) (layer "F.Cu") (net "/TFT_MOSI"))
 (segment (start 98.3442 131.2958) (end 98.3442 133.1927) (width 0.2) (layer "F.Cu") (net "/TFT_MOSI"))
 (segment (start 99.5 130.14) (end 98.3442 131.2958) (width 0.2) (layer "F.Cu") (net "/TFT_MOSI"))
 (segment (start 98.3442 133.1927) (end 99.2198 134.0683) (width 0.2) (layer "F.Cu") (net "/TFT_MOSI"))
 (segment (start 99.2198 134.0683) (end 100.0326 134.0683) (width 0.2) (layer "F.Cu") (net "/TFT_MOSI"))
 (segment (start 108.4 141.58) (end 108.4 154.41) (width 0.2) (layer "F.Cu") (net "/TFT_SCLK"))
 (segment (start 99.5 132.68) (end 108.4 141.58) (width 0.2) (layer "F.Cu") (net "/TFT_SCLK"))
 (segment (start 78.2978 128.14) (end 92.42 128.14) (width 0.2) (layer "B.Cu") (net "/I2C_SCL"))
 (segment (start 78.72 124.33) (end 77.5259 125.5241) (width 0.2) (layer "B.Cu") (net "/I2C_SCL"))
 (segment (start 77.5259 125.5241) (end 77.5259 127.3681) (width 0.2) (layer "B.Cu") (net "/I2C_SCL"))
 (segment (start 77.5259 127.3681) (end 78.2978 128.14) (width 0.2) (layer "B.Cu") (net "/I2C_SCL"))
 (segment (start 92.42 128.14) (end 99.5 135.22) (width 0.2) (layer "B.Cu") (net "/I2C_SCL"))
 (segment (start 104.5411 142.8011) (end 104.5411 160.3713) (width 0.2) (layer "F.Cu") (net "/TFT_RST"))
 (segment (start 104.5411 160.3713) (end 105.7492 161.5794) (width 0.2) (layer "F.Cu") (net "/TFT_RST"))
 (segment (start 105.7492 161.5794) (end 111.9006 161.5794) (width 0.2) (layer "F.Cu") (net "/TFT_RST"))
 (segment (start 111.9006 161.5794) (end 113.48 160) (width 0.2) (layer "F.Cu") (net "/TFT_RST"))
 (segment (start 99.5 137.76) (end 104.5411 142.8011) (width 0.2) (layer "F.Cu") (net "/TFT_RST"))
 (segment (start 78.72 126.87) (end 91.8824 113.7076) (width 0.2) (layer "B.Cu") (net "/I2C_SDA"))
 (segment (start 121.0124 113.7076) (end 122.36 112.36) (width 0.2) (layer "B.Cu") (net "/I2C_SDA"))
 (segment (start 91.8824 113.7076) (end 121.0124 113.7076) (width 0.2) (layer "B.Cu") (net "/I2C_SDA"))
 (segment (start 80.5 127.63) (end 80.5 99.3) (width 1) (layer "F.Cu") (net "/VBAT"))
 (segment (start 80.5 99.3) (end 77.45 96.25) (width 1) (layer "F.Cu") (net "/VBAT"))
 (segment (start 83 90.7) (end 83 82.5) (width 1) (layer "F.Cu") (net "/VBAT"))
 (segment (start 77.45 96.25) (end 83 90.7) (width 1) (layer "F.Cu") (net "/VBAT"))
 (segment (start 78.72 129.41) (end 80.5 127.63) (width 1) (layer "F.Cu") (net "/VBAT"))
 (segment (start 91.9694 142.6755) (end 91.9694 158.8094) (width 0.2) (layer "F.Cu") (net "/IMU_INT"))
 (segment (start 91.9694 158.8094) (end 93.16 160) (width 0.2) (layer "F.Cu") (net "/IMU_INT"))
 (via (at 91.9694 142.6755) (size 0.8) (drill 0.4) (layers "F.Cu" "B.Cu") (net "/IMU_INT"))
 (segment (start 101.562 134.857) (end 99.929 136.49) (width 0.2) (layer "B.Cu") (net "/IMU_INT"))
 (segment (start 122.36 97.12) (end 123.5235 98.2835) (width 0.2) (layer "B.Cu") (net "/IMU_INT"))
 (segment (start 123.5235 98.2835) (end 123.5235 112.8316) (width 0.2) (layer "B.Cu") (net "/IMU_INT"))
 (segment (start 121.8496 113.7483) (end 101.562 134.0359) (width 0.2) (layer "B.Cu") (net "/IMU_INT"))
 (segment (start 98.1549 136.49) (end 91.9694 142.6755) (width 0.2) (layer "B.Cu") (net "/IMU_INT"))
 (segment (start 99.929 136.49) (end 98.1549 136.49) (width 0.2) (layer "B.Cu") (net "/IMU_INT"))
 (segment (start 122.6068 113.7483) (end 121.8496 113.7483) (width 0.2) (layer "B.Cu") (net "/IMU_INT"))
 (segment (start 123.5235 112.8316) (end 122.6068 113.7483) (width 0.2) (layer "B.Cu") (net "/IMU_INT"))
 (segment (start 101.562 134.0359) (end 101.562 134.857) (width 0.2) (layer "B.Cu") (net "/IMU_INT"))
 (segment (start 106.8462 115.1738) (end 122.36 99.66) (width 0.2) (layer "F.Cu") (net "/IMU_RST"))
 (segment (start 106.9212 134.2058) (end 106.8462 115.1738) (width 0.2) (layer "F.Cu") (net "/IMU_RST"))
 (via (at 106.9212 134.2058) (size 0.8) (drill 0.4) (layers "F.Cu" "B.Cu") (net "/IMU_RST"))
 (segment (start 93.16 154.41) (end 106.8462 140.7238) (width 0.2) (layer "B.Cu") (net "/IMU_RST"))
 (segment (start 106.8462 140.7238) (end 106.9212 134.2058) (width 0.2) (layer "B.Cu") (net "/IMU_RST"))
 (segment (start 110.75 113.81) (end 110.75 138) (width 0.2) (layer "F.Cu") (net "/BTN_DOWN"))
 (segment (start 122.36 102.2) (end 110.75 113.81) (width 0.2) (layer "F.Cu") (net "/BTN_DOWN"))
 (segment (start 103.75 153.98) (end 103.32 154.41) (width 0.2) (layer "F.Cu") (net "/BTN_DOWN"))
 (segment (start 103.75 146) (end 103.75 153.98) (width 0.2) (layer "F.Cu") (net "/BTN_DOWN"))
 (via (at 110.75 138) (size 0.8) (drill 0.4) (layers "F.Cu" "B.Cu") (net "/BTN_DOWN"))
 (via (at 103.75 146) (size 0.8) (drill 0.4) (layers "F.Cu" "B.Cu") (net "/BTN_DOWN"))
 (segment (start 110.75 138) (end 110.75 139) (width 0.2) (layer "B.Cu") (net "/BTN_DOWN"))
 (segment (start 110.75 139) (end 103.75 146) (width 0.2) (layer "B.Cu") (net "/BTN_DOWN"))
 (segment (start 123.5604 125.5094) (end 123.5604 105.9404) (width 0.2) (layer "F.Cu") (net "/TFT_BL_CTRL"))
 (segment (start 122.7398 126.33) (end 123.5604 125.5094) (width 0.2) (layer "F.Cu") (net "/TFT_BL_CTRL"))
 (segment (start 121.9695 126.33) (end 122.7398 126.33) (width 0.2) (layer "F.Cu") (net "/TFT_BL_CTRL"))
 (segment (start 113.48 134.8195) (end 121.9695 126.33) (width 0.2) (layer "F.Cu") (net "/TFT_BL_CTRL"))
 (segment (start 123.5604 105.9404) (end 122.36 104.74) (width 0.2) (layer "F.Cu") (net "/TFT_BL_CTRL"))
 (segment (start 113.48 154.41) (end 113.48 134.8195) (width 0.2) (layer "F.Cu") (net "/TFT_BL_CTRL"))
 (segment (start 112.1 117.54) (end 112.1 160.476) (width 0.2) (layer "F.Cu") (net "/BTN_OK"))
 (segment (start 122.36 107.28) (end 112.1 117.54) (width 0.2) (layer "F.Cu") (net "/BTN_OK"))
 (segment (start 111.4006 161.1754) (end 107.0354 161.1754) (width 0.2) (layer "F.Cu") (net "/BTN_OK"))
 (segment (start 107.0354 161.1754) (end 105.86 160) (width 0.2) (layer "F.Cu") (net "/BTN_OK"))
 (segment (start 112.1 160.476) (end 111.4006 161.1754) (width 0.2) (layer "F.Cu") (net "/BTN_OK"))
 (segment (start 105.5 154.05) (end 105.86 154.41) (width 0.2) (layer "F.Cu") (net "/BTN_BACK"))
 (segment (start 113 119.18) (end 113 127) (width 0.2) (layer "F.Cu") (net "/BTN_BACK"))
 (segment (start 105.5 141) (end 105.5 154.05) (width 0.2) (layer "F.Cu") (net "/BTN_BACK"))
 (segment (start 122.36 109.82) (end 113 119.18) (width 0.2) (layer "F.Cu") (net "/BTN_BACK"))
 (via (at 105.5 141) (size 0.8) (drill 0.4) (layers "F.Cu" "B.Cu") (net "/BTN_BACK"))
 (via (at 113 127) (size 0.8) (drill 0.4) (layers "F.Cu" "B.Cu") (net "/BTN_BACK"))
 (segment (start 113 127) (end 105.5 134.5) (width 0.2) (layer "B.Cu") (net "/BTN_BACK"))
 (segment (start 105.5 134.5) (end 105.5 141) (width 0.2) (layer "B.Cu") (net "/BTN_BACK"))
 (segment (start 120.9701 157.5899) (end 120.9701 128.9898) (width 0.2) (layer "F.Cu") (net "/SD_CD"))
 (segment (start 120.9702 128.9898) (end 122.36 127.6) (width 0.2) (layer "F.Cu") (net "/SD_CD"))
 (segment (start 118.56 160) (end 120.9701 157.5899) (width 0.2) (layer "F.Cu") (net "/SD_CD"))
 (segment (start 120.9701 128.9898) (end 120.9702 128.9898) (width 0.2) (layer "F.Cu") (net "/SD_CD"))
 (segment (start 117.29 152.5003) (end 117.29 154.7704) (width 0.2) (layer "B.Cu") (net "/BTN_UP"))
 (segment (start 122.36 130.14) (end 123.5237 131.3037) (width 0.2) (layer "B.Cu") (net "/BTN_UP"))
 (segment (start 117.29 154.7704) (end 114.276 157.7844) (width 0.2) (layer "B.Cu") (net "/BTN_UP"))
 (segment (start 105.5356 157.7844) (end 103.32 160) (width 0.2) (layer "B.Cu") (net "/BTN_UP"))
 (segment (start 114.276 157.7844) (end 105.5356 157.7844) (width 0.2) (layer "B.Cu") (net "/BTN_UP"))
 (segment (start 123.5237 146.2666) (end 117.29 152.5003) (width 0.2) (layer "B.Cu") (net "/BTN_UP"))
 (segment (start 123.5237 131.3037) (end 123.5237 146.2666) (width 0.2) (layer "B.Cu") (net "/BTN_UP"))
 (segment (start 122.36 132.68) (end 118.2954 132.68) (width 0.2) (layer "B.Cu") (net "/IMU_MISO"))
 (segment (start 89.2898 155.6198) (end 88.08 154.41) (width 0.2) (layer "B.Cu") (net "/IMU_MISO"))
 (segment (start 96.8517 154.1237) (end 96.8517 154.8871) (width 0.2) (layer "B.Cu") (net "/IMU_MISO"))
 (segment (start 118.2954 132.68) (end 96.8517 154.1237) (width 0.2) (layer "B.Cu") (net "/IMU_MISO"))
 (segment (start 96.8517 154.8871) (end 96.119 155.6198) (width 0.2) (layer "B.Cu") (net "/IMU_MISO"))
 (segment (start 96.119 155.6198) (end 89.2898 155.6198) (width 0.2) (layer "B.Cu") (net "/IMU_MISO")))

